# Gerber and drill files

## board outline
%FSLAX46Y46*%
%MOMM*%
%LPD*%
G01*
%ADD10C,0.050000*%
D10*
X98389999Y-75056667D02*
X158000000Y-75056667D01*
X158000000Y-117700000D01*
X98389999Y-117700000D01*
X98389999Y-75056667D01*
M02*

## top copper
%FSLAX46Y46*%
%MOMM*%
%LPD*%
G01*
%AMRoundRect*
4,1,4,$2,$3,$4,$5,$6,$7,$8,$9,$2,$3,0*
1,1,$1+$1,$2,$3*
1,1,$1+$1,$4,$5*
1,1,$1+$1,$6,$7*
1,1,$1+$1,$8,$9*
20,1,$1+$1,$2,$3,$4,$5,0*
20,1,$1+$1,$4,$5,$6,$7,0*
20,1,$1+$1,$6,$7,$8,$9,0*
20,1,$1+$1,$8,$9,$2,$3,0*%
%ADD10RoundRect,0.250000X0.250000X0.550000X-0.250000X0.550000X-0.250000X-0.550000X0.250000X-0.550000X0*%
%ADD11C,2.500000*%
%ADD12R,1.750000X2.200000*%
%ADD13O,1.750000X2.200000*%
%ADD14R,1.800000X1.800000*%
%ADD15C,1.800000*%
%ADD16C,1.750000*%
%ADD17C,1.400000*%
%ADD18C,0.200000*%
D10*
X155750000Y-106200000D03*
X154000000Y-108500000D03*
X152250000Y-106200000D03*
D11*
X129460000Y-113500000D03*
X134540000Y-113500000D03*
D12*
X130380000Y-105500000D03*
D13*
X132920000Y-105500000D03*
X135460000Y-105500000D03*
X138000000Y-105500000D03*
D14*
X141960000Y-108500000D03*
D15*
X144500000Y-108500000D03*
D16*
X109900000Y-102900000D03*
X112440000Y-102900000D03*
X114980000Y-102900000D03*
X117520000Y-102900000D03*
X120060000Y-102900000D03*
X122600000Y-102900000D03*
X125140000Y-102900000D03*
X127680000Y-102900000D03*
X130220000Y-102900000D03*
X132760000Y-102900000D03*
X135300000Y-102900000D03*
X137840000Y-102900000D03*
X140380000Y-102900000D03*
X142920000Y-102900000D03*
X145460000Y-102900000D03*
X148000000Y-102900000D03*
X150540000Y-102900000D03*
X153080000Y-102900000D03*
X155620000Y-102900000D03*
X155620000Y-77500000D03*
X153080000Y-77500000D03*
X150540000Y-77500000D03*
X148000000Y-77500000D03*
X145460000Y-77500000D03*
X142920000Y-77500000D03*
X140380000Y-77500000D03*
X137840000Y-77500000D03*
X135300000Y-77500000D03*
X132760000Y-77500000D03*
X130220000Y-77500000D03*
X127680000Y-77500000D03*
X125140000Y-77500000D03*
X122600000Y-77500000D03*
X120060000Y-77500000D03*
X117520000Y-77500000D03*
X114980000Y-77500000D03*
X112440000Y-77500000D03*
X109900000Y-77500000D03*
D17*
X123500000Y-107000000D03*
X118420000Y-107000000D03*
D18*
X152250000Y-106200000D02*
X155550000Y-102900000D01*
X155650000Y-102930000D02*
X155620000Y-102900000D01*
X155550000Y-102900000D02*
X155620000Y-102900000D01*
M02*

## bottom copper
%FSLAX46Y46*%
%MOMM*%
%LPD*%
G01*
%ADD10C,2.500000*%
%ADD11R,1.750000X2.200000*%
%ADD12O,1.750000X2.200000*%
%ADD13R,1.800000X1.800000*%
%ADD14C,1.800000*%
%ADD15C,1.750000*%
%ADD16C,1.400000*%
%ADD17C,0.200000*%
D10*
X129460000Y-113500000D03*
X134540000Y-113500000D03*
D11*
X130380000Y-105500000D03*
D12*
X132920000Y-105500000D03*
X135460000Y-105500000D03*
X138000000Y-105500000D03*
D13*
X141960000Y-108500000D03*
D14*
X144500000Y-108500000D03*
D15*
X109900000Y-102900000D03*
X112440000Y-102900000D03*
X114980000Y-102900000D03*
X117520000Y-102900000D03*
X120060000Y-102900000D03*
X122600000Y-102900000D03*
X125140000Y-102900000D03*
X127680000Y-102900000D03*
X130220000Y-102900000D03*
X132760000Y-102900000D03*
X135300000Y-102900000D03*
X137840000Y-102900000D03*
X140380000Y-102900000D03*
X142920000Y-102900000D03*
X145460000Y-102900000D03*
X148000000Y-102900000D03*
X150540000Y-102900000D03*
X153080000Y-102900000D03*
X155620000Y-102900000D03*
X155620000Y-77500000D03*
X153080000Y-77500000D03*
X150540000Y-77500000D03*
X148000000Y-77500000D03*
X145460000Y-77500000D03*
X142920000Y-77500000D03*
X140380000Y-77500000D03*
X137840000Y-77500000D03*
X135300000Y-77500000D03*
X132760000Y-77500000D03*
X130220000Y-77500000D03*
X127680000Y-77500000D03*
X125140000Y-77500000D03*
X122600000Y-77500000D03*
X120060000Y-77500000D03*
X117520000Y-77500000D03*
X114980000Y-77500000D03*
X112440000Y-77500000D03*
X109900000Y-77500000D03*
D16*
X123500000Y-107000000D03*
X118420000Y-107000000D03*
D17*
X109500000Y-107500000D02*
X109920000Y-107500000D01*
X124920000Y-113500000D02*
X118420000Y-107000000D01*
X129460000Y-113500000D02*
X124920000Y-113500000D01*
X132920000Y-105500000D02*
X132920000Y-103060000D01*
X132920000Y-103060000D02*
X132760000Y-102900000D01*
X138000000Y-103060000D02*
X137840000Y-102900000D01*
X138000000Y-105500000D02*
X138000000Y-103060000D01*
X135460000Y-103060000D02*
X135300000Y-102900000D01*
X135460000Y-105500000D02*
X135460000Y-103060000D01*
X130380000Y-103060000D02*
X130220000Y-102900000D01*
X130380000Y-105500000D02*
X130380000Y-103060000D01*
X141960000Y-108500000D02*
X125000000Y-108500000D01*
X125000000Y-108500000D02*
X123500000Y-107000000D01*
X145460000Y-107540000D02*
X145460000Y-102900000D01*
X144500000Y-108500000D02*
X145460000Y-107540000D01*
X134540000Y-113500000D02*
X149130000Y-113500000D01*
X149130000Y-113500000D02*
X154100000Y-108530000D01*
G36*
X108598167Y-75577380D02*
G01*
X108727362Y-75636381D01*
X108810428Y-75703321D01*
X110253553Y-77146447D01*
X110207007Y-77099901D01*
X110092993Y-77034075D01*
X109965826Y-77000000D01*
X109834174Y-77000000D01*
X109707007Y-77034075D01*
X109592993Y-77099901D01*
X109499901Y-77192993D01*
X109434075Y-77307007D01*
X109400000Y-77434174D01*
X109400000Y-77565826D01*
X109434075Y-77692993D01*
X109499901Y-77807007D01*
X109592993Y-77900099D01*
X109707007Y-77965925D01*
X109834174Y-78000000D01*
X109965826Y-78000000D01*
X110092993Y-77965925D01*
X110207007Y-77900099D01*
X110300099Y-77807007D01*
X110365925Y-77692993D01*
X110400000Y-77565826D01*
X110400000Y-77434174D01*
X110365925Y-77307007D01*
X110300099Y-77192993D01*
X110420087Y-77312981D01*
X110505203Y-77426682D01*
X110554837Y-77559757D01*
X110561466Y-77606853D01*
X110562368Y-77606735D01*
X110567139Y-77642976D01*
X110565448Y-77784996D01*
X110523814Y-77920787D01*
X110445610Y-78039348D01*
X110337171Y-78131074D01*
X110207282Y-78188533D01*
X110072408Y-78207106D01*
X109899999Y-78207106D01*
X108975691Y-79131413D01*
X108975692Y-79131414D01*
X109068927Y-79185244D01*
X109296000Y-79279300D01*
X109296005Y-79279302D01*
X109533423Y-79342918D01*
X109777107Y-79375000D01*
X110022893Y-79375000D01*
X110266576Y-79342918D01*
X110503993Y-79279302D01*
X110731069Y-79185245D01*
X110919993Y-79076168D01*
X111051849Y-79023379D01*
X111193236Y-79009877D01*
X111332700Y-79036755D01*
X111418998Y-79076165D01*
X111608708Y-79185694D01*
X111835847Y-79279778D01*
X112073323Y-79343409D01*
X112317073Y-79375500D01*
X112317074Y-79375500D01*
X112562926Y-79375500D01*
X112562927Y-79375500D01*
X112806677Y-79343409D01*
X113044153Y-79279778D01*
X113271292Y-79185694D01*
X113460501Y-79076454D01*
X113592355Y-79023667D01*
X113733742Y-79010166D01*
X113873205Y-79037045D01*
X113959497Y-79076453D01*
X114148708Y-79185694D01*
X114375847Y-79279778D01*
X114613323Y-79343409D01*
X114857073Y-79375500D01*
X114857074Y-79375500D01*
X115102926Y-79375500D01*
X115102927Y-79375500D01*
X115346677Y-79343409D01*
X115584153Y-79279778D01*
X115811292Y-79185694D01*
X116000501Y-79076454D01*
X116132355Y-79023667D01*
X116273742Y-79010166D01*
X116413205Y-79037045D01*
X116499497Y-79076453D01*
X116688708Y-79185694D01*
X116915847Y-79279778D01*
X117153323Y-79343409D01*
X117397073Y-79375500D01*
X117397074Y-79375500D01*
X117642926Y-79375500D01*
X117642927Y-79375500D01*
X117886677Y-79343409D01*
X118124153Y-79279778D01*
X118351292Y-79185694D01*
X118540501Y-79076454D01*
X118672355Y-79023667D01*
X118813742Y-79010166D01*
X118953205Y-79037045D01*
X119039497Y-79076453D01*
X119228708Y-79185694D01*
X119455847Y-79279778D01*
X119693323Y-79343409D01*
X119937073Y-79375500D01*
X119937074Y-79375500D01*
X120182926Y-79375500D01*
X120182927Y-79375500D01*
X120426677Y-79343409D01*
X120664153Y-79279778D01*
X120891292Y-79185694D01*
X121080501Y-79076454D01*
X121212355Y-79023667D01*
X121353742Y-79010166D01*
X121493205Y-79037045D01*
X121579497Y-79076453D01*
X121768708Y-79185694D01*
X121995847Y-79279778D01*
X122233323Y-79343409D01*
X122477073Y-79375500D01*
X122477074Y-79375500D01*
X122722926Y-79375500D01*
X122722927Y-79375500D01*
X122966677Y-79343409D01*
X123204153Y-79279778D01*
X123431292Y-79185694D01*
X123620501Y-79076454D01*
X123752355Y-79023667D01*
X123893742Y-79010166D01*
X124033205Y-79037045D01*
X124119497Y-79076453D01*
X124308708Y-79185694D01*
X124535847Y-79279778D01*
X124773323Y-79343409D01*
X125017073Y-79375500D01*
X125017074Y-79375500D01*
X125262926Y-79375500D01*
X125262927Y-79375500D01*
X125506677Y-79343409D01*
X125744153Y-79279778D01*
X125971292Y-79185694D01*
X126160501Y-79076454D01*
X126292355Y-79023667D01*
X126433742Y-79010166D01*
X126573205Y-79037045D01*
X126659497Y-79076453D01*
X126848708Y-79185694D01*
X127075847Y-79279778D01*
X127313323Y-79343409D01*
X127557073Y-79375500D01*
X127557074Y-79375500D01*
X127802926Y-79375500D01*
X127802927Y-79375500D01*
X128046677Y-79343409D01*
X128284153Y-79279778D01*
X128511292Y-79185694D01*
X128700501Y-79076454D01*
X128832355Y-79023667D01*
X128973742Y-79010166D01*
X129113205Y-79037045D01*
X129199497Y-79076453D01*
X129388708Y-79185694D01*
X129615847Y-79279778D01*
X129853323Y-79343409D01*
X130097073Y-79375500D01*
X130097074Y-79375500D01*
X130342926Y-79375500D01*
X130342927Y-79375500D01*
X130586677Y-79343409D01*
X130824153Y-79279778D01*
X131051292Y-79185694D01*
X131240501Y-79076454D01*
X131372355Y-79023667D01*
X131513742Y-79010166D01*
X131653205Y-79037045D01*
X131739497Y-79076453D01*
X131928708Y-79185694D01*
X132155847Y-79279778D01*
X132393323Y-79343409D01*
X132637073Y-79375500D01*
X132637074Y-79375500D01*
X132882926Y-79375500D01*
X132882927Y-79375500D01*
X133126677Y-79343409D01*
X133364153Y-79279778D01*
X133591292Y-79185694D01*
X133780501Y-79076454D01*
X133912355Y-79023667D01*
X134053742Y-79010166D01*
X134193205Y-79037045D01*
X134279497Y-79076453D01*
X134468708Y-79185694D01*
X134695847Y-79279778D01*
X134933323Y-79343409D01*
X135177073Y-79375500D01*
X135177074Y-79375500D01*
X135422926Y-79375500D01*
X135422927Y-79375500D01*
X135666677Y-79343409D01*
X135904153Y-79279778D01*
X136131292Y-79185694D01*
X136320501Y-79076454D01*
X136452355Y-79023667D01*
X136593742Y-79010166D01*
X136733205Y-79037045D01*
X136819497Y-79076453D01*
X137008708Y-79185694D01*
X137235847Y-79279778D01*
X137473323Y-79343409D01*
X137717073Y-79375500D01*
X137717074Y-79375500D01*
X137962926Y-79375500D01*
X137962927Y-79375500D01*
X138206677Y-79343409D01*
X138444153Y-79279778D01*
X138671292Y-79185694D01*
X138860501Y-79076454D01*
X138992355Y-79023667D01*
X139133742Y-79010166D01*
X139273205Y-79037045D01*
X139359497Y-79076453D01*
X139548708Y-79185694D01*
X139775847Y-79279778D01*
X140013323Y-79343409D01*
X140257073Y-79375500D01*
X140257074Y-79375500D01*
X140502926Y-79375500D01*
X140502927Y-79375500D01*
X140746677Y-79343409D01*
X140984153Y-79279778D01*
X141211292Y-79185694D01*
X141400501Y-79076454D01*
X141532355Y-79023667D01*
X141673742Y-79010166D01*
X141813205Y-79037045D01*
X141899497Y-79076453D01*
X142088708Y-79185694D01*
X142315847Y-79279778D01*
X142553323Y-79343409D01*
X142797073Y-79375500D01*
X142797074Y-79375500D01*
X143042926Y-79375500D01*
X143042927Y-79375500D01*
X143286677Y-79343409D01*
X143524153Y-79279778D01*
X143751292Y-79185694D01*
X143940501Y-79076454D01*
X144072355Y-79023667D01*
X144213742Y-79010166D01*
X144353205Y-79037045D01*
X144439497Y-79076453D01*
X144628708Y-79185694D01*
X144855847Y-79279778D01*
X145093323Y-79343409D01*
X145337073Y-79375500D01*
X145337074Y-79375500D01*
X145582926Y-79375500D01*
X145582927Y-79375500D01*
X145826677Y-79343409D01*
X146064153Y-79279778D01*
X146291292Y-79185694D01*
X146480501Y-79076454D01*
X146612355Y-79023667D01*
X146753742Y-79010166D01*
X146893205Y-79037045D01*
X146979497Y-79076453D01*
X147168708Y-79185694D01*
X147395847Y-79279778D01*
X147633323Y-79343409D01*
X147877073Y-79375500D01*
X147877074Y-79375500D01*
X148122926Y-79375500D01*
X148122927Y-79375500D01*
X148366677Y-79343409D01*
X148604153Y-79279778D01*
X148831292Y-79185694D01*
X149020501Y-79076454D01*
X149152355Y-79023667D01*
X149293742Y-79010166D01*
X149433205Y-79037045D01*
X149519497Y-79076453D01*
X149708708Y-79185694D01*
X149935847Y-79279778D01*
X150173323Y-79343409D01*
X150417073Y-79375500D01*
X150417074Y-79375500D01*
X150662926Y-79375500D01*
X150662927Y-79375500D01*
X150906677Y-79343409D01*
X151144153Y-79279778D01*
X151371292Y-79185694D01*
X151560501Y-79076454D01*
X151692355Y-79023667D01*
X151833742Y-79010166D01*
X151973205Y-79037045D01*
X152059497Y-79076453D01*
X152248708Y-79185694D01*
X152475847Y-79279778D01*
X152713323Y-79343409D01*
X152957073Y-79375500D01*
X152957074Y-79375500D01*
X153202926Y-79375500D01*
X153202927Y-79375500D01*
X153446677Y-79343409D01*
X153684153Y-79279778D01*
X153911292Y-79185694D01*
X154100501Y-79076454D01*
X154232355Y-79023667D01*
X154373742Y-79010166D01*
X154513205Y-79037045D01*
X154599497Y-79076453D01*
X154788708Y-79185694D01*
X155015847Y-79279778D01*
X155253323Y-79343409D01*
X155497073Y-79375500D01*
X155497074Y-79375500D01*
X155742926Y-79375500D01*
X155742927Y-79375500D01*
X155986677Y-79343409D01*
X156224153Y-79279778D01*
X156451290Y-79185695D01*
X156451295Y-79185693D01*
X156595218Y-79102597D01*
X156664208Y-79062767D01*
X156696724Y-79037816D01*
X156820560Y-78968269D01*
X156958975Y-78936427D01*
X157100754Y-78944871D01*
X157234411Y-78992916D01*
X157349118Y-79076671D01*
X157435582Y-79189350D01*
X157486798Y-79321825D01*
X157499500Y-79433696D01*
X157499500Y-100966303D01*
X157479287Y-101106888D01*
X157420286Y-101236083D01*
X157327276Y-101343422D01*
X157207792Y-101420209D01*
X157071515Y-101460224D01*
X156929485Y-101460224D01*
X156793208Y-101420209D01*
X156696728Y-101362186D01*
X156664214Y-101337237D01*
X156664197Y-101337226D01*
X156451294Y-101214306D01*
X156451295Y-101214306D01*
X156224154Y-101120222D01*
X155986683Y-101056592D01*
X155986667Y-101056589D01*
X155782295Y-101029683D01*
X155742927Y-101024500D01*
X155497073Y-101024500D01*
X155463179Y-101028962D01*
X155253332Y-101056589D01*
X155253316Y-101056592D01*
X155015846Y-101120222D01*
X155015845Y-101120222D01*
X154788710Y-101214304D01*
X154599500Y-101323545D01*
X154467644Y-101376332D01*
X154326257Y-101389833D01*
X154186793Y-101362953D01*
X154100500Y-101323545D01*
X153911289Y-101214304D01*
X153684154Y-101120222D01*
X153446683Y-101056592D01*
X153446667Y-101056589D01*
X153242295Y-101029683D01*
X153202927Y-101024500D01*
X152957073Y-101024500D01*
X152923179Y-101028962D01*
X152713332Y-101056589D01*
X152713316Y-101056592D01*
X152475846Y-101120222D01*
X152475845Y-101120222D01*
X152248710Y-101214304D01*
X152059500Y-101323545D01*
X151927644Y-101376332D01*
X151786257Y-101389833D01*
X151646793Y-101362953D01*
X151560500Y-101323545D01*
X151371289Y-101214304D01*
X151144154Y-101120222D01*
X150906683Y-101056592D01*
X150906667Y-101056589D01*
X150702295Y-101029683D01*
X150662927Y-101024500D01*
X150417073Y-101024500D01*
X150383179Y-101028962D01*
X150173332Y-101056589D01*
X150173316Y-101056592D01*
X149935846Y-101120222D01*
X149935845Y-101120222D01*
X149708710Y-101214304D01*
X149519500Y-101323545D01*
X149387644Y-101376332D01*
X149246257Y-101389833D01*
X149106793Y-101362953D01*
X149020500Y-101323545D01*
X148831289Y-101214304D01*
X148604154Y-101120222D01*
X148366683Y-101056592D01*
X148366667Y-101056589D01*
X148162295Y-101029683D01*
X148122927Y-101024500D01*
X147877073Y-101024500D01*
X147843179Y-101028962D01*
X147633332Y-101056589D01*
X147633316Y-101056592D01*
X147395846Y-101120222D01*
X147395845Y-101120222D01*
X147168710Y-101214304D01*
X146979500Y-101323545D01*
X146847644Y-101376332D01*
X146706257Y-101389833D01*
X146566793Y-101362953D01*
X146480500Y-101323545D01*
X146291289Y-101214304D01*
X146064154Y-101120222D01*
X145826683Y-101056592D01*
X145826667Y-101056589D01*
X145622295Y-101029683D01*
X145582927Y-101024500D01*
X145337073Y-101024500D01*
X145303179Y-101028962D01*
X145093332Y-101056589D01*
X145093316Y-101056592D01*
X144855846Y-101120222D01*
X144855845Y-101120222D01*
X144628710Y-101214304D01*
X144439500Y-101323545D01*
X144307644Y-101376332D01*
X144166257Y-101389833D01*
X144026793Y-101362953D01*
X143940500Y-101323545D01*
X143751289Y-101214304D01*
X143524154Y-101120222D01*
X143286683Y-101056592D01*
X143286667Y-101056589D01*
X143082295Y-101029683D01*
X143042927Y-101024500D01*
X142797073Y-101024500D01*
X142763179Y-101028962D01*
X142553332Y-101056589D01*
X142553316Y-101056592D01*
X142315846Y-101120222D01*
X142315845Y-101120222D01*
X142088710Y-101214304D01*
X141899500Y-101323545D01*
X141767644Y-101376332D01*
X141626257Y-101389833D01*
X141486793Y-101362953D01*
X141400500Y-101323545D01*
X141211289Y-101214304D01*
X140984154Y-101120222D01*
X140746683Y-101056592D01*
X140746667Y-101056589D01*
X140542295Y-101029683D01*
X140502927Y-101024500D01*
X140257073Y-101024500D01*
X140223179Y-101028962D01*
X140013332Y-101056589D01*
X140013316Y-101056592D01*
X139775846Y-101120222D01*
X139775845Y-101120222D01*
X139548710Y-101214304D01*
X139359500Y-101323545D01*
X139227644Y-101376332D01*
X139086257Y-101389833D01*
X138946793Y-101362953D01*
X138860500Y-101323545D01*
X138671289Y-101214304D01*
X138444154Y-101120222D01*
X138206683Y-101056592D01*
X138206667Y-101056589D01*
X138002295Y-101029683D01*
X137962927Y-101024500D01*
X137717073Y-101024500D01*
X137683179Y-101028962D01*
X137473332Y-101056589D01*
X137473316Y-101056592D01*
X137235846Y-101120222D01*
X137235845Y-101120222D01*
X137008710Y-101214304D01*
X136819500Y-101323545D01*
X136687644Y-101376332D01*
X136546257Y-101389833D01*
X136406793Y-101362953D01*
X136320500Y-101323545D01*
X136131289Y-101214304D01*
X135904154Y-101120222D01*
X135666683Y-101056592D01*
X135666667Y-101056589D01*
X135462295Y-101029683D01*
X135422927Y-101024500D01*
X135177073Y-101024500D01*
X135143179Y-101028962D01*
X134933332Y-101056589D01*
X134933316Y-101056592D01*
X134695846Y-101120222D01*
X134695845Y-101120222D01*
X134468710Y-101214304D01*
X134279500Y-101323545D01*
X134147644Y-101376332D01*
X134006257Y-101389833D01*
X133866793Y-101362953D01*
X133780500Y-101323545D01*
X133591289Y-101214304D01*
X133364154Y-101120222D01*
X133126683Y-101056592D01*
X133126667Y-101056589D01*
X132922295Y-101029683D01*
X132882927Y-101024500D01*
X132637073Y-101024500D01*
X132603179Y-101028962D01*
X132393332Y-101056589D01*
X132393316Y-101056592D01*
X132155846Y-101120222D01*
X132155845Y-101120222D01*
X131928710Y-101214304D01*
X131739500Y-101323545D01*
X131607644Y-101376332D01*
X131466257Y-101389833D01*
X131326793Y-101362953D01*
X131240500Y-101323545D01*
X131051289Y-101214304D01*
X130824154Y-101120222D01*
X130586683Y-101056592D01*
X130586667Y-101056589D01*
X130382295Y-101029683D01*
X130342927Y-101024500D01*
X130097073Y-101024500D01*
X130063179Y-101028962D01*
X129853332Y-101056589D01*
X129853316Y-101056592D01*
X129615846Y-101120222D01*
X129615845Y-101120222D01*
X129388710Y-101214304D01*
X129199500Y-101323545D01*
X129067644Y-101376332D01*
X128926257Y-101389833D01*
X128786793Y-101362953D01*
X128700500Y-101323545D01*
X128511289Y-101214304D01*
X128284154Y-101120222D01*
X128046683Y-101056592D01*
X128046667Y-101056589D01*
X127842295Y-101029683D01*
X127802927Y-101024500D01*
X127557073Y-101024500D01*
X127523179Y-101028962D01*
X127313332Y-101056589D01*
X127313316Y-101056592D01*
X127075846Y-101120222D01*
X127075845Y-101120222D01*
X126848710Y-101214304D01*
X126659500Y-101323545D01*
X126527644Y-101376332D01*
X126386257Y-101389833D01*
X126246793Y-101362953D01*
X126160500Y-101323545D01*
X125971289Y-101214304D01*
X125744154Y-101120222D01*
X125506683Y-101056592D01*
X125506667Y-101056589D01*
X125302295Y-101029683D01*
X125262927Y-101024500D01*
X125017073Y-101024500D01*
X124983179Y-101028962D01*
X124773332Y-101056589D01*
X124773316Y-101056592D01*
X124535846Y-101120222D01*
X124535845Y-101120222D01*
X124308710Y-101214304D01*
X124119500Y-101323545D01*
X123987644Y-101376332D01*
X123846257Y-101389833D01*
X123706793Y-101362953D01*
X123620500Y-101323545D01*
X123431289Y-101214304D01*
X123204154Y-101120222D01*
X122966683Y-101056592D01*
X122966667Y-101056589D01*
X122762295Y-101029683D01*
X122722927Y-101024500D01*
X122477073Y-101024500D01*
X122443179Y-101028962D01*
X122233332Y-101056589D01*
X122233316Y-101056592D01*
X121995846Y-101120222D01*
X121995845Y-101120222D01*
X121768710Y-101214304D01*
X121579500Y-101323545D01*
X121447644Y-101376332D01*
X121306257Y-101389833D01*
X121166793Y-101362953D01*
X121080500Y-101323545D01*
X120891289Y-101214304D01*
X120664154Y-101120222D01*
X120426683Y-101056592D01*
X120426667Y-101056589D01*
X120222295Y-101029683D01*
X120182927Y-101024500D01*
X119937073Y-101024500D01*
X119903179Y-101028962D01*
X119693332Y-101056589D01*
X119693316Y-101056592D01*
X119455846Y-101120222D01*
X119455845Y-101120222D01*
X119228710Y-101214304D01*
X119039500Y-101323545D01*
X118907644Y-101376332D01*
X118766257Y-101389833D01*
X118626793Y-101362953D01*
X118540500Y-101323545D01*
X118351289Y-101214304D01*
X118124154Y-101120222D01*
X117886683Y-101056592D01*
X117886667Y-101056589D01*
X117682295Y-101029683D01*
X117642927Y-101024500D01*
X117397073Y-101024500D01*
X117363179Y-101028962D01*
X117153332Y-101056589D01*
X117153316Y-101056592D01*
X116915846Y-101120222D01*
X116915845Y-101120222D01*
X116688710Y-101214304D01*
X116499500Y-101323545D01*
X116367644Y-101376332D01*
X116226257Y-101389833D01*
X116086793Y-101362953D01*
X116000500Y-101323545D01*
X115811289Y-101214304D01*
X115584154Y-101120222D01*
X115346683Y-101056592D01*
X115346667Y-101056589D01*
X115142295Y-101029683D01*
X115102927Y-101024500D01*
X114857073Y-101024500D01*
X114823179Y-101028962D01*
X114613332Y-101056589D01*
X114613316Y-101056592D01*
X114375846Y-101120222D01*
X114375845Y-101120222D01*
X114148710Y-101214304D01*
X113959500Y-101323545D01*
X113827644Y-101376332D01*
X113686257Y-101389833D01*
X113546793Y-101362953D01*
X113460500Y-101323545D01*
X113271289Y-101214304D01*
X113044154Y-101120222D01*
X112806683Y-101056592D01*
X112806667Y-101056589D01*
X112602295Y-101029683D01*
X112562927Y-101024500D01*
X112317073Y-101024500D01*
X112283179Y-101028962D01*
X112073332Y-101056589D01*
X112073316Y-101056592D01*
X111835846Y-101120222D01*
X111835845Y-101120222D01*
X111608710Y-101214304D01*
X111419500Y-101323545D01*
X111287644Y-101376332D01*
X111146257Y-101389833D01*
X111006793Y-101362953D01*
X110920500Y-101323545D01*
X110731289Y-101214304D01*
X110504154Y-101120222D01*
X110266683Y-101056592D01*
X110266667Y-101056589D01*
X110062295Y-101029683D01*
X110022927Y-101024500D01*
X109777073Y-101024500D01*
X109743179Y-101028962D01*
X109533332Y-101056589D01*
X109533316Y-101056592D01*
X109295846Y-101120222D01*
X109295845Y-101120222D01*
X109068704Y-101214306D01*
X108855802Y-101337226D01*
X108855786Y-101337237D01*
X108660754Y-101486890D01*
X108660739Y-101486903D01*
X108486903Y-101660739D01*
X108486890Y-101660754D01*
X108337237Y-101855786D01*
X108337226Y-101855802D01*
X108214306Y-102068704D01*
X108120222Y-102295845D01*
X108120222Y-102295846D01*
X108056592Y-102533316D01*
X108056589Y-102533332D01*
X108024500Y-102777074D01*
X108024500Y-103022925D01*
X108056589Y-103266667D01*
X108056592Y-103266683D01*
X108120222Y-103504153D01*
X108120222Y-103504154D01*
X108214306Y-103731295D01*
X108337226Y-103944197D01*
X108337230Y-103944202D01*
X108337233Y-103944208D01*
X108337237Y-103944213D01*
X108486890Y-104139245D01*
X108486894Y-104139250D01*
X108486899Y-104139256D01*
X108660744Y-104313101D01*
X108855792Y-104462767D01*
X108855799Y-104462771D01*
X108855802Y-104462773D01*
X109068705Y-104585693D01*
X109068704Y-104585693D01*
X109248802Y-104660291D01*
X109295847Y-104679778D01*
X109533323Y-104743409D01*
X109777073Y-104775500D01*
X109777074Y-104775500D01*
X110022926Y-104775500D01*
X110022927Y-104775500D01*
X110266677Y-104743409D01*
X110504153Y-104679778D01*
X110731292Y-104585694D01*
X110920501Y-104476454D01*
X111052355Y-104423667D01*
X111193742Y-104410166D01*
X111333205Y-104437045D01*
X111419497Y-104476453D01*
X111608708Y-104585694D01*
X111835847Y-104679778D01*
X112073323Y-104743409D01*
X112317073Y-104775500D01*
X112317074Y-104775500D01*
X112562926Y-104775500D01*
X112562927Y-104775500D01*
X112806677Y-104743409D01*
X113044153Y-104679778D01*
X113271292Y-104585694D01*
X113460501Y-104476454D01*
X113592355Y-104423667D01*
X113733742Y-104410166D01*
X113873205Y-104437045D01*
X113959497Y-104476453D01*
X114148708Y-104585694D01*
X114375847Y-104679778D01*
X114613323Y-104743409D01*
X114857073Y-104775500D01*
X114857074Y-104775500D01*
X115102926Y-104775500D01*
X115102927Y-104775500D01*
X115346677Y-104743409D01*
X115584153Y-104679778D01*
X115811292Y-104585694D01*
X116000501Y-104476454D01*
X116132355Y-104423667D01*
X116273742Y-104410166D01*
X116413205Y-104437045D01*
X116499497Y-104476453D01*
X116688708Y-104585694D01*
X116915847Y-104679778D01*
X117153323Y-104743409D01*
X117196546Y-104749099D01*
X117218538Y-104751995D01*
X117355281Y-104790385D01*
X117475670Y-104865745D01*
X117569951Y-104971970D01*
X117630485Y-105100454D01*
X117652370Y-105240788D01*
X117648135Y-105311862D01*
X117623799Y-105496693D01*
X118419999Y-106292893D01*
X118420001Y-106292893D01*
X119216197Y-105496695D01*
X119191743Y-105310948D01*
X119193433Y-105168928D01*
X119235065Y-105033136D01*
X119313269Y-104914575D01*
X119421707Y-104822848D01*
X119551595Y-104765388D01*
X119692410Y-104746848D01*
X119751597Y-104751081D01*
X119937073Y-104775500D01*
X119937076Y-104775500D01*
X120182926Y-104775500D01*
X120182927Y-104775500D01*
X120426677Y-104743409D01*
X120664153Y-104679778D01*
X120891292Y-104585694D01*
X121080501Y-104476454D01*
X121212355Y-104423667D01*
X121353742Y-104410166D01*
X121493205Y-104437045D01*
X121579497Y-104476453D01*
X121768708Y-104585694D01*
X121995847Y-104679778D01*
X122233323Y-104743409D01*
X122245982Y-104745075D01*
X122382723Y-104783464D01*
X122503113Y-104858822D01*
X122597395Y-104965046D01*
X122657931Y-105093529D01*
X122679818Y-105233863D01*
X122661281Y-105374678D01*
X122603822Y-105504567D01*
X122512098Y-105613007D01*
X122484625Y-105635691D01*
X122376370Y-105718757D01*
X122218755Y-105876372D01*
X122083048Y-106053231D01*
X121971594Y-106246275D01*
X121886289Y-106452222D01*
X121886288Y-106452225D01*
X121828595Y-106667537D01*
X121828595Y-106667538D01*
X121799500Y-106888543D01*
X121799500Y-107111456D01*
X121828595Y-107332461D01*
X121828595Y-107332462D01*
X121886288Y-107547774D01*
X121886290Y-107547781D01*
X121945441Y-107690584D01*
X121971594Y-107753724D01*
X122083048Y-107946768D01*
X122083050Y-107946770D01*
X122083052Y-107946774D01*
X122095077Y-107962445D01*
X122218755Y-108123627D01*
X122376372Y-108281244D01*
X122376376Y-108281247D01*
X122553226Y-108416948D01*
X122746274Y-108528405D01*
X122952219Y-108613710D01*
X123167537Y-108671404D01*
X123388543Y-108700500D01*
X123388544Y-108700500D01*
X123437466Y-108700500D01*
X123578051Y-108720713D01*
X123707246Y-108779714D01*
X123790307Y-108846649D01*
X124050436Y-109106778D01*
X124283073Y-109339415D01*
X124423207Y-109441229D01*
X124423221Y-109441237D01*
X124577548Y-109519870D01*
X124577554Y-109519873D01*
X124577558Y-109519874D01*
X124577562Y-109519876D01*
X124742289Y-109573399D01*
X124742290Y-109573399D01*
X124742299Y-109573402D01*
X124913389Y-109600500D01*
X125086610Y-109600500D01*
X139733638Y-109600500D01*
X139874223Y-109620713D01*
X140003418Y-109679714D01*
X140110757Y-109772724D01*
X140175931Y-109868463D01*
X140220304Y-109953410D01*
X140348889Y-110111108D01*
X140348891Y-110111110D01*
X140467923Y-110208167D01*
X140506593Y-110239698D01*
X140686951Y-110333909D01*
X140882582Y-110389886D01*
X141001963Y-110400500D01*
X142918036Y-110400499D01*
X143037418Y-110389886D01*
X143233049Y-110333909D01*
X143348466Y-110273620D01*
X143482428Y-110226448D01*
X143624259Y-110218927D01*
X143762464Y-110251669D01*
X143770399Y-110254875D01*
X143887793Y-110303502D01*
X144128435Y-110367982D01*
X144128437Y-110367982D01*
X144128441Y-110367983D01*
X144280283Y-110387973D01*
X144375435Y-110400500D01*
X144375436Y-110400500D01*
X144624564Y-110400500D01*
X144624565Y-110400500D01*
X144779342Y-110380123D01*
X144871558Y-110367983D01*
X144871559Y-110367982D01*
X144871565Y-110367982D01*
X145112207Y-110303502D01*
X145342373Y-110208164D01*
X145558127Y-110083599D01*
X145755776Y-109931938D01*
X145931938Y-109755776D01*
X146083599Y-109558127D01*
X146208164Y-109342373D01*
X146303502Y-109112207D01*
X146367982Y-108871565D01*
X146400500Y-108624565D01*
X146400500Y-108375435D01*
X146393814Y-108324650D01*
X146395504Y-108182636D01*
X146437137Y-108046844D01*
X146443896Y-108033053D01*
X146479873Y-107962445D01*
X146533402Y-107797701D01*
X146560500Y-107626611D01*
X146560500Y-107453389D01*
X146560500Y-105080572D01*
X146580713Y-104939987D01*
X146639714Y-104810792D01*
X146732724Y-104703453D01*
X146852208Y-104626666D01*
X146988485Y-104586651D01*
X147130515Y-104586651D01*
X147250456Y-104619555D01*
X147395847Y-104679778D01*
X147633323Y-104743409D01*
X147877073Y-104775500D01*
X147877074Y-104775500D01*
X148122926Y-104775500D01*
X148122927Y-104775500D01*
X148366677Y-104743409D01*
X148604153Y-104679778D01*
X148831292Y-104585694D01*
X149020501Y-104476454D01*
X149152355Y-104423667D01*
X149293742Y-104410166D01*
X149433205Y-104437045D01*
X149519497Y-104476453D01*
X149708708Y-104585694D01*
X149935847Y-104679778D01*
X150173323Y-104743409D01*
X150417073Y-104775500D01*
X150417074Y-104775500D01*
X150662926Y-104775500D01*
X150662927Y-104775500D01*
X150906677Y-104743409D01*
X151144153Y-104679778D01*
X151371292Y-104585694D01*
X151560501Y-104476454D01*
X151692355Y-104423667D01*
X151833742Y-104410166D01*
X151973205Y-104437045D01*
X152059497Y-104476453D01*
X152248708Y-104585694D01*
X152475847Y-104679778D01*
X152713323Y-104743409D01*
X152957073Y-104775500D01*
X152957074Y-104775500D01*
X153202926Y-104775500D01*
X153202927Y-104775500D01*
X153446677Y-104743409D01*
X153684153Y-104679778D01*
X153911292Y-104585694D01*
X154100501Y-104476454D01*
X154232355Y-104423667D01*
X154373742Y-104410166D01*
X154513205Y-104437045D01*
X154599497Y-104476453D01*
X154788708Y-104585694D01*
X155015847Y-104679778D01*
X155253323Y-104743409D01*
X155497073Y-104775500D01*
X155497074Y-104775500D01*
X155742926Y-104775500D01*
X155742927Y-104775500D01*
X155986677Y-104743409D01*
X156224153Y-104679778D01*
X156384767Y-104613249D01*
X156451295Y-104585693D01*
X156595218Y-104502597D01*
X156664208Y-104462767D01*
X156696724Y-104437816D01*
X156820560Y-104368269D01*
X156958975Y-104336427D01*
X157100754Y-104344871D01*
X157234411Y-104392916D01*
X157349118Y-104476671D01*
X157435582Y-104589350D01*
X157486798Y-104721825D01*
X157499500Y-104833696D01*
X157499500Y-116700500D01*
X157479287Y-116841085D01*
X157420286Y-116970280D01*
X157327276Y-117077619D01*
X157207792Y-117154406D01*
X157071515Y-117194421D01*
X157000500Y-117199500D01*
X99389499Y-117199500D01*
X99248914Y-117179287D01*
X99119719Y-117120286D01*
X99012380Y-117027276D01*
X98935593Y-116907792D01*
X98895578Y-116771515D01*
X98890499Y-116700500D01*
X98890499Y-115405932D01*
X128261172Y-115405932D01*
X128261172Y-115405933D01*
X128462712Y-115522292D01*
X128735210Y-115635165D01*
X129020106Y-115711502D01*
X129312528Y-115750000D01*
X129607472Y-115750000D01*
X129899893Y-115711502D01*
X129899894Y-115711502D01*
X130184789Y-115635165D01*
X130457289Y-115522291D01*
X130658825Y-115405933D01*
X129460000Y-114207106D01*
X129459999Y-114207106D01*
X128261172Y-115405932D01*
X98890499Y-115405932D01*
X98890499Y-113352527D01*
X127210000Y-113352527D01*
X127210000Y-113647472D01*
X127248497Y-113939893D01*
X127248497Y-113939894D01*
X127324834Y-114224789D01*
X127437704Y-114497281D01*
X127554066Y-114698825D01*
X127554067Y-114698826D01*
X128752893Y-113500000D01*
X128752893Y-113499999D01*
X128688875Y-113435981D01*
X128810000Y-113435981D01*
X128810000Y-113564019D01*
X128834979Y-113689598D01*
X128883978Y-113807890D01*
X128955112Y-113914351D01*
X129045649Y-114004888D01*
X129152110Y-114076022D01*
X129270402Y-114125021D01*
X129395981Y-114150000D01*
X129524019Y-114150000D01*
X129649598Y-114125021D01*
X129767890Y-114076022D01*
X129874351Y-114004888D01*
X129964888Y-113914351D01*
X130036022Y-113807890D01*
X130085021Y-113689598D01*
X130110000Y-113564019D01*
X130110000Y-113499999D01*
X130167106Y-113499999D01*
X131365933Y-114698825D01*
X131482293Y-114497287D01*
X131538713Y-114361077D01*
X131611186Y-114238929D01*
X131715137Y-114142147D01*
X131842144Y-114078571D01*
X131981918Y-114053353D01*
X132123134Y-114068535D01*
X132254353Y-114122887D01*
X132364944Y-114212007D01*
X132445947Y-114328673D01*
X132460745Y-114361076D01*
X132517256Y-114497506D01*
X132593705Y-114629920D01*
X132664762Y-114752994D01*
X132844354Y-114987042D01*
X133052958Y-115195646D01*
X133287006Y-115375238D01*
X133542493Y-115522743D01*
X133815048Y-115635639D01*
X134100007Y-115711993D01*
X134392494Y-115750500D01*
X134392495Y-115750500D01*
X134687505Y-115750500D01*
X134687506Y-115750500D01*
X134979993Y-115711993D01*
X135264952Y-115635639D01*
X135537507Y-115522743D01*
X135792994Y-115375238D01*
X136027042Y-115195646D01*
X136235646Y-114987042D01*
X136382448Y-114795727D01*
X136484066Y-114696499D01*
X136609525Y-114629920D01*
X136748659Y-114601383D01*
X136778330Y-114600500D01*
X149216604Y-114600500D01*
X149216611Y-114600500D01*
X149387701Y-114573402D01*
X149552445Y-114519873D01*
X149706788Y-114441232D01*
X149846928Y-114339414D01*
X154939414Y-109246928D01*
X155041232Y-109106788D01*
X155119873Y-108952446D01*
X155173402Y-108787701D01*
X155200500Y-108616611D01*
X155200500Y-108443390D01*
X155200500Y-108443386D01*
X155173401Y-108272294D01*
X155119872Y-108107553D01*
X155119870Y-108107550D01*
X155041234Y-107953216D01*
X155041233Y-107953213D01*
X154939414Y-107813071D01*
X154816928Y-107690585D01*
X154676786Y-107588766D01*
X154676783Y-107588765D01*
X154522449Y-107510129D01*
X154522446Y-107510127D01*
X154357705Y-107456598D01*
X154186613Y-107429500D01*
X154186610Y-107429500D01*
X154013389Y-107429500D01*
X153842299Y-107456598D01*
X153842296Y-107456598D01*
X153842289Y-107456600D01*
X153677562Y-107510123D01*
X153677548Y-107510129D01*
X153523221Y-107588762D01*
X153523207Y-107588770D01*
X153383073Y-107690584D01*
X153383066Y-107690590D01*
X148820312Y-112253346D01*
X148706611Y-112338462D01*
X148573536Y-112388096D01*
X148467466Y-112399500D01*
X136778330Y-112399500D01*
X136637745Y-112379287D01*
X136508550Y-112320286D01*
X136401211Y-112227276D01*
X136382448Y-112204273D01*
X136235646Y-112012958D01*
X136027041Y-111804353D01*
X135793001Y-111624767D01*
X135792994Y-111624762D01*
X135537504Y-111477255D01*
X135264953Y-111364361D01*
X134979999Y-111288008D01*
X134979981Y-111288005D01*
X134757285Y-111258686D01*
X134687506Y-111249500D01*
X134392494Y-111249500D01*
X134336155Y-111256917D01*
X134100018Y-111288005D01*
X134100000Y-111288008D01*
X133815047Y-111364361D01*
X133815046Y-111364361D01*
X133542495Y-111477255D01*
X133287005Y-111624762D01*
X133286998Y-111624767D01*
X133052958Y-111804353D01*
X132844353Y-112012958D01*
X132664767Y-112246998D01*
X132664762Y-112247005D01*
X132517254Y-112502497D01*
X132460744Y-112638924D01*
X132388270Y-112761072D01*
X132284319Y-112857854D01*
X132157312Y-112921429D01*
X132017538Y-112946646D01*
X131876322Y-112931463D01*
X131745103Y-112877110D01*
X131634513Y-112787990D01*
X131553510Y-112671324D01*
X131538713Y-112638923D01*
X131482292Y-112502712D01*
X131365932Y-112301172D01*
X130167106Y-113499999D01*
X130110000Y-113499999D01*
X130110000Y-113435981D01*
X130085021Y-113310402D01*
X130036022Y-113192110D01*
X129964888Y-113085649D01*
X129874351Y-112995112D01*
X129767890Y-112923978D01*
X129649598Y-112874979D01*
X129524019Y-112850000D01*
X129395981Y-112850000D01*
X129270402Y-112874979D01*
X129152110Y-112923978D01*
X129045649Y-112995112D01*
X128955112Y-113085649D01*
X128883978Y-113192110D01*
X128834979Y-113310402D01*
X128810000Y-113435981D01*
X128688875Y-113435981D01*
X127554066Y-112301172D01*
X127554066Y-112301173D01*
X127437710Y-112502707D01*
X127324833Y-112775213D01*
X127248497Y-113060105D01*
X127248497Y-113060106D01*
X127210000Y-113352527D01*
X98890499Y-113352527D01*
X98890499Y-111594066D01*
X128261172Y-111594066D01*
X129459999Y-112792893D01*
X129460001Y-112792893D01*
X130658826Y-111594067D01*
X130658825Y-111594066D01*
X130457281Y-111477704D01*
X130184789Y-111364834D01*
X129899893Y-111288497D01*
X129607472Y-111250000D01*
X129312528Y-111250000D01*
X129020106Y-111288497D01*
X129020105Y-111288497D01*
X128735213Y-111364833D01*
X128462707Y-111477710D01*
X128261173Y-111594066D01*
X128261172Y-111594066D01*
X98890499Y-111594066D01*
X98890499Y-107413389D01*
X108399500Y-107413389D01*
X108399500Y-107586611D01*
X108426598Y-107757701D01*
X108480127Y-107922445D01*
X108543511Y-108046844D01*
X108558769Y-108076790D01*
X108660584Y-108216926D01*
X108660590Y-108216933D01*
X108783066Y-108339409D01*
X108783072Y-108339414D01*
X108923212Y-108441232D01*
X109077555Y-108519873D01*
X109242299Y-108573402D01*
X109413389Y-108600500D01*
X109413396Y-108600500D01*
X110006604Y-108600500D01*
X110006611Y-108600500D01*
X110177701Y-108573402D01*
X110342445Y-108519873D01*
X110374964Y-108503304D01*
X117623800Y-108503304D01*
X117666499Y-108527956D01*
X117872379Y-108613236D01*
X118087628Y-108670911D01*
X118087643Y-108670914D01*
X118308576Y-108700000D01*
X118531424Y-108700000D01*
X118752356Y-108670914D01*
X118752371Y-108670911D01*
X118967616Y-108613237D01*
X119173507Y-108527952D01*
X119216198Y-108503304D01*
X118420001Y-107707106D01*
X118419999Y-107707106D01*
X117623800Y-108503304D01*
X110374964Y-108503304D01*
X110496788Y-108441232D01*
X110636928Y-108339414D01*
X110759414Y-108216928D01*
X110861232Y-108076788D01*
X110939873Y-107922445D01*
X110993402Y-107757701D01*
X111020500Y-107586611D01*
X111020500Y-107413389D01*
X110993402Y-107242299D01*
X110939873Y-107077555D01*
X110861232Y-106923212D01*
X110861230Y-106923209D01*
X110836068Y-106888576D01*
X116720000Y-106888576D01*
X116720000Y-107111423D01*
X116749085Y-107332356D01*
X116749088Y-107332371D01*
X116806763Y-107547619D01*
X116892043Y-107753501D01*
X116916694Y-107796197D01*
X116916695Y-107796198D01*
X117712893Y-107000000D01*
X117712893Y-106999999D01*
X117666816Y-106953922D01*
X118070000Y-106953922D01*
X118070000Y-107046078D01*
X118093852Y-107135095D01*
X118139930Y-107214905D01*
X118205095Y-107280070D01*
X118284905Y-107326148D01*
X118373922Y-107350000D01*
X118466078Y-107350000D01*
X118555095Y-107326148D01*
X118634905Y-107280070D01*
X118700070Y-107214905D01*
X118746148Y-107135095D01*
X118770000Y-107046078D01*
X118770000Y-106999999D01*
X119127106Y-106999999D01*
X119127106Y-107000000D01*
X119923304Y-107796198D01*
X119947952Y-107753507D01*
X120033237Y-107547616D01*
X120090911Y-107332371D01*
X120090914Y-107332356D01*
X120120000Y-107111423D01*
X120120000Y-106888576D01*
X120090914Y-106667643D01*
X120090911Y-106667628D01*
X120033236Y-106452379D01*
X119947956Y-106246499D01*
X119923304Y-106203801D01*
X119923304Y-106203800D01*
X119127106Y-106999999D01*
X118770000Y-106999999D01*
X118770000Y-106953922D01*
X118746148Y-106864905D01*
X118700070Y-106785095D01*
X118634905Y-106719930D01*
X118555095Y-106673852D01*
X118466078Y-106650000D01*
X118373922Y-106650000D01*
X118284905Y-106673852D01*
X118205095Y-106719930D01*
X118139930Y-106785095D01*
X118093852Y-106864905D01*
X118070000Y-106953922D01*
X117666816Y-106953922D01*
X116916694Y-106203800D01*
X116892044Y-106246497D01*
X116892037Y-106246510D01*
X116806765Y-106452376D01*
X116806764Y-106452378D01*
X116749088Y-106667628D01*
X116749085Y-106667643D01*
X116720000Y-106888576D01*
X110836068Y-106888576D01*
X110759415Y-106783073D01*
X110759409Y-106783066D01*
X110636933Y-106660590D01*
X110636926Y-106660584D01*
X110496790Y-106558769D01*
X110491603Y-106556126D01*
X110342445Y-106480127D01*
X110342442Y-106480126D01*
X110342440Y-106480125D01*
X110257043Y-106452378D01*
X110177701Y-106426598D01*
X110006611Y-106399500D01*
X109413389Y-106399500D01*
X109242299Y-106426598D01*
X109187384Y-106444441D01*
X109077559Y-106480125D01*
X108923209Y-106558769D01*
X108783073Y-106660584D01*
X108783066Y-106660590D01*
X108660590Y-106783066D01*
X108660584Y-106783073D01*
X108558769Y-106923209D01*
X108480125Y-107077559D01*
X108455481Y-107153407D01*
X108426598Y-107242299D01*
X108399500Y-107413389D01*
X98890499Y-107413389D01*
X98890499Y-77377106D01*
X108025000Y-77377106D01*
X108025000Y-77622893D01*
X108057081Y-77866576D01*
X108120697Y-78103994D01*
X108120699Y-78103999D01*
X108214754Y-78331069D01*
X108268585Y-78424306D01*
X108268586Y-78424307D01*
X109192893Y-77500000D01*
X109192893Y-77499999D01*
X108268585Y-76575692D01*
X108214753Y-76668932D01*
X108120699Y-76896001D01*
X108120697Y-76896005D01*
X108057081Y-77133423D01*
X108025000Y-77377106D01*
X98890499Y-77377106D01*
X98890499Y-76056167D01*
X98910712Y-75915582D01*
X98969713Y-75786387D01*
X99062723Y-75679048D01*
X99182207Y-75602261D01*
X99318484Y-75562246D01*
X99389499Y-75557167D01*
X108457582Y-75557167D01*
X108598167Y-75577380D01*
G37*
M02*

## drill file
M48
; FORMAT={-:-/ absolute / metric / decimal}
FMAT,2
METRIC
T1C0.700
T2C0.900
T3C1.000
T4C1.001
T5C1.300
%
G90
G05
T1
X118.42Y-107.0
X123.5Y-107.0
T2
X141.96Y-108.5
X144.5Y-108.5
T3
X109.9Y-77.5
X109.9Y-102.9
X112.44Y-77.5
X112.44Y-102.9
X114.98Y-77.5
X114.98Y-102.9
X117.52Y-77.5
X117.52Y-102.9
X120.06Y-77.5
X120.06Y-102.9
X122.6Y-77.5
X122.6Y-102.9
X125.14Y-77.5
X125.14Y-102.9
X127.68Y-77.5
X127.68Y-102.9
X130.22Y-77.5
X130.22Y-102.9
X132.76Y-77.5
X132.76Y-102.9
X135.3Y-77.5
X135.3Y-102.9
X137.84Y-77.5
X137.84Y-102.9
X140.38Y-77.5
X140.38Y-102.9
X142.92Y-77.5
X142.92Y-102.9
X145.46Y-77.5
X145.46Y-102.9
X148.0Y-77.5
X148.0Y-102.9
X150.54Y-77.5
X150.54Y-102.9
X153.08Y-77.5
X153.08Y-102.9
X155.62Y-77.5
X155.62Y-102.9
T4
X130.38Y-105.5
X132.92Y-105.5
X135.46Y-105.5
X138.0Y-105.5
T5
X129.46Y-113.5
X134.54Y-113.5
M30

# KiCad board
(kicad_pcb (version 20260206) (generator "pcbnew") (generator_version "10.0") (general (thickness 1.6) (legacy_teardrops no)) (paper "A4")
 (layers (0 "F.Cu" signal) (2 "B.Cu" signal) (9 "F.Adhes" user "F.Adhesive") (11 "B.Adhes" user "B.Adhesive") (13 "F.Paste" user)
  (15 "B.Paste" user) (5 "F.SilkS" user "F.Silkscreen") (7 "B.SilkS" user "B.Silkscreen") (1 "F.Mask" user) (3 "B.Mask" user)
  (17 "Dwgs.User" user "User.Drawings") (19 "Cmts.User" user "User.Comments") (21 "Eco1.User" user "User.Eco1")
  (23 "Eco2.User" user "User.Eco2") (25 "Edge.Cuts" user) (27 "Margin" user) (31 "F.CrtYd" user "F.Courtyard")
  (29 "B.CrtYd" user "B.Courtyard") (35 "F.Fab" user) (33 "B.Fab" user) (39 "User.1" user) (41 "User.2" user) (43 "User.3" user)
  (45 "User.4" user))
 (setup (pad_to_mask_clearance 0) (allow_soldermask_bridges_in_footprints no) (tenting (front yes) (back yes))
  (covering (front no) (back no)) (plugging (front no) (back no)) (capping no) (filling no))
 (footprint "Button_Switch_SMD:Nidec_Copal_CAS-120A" (layer "F.Cu") (at 154 107.35 -90)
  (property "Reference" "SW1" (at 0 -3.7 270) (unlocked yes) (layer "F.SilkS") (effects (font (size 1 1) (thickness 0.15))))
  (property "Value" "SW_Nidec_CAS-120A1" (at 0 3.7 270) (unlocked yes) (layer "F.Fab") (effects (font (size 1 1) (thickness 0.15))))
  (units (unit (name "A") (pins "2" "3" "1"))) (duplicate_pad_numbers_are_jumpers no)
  (pad "1" smd roundrect (at -1.15 -1.75 180) (size 1 1.6) (layers "F.Cu" "F.Mask" "F.Paste") (roundrect_rratio 0.25)
   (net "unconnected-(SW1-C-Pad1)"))
  (pad "2" smd roundrect (at 1.15 0 180) (size 1 1.6) (layers "F.Cu" "F.Mask" "F.Paste") (roundrect_rratio 0.25) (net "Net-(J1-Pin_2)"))
  (pad "3" smd roundrect (at -1.15 1.75 180) (size 1 1.6) (layers "F.Cu" "F.Mask" "F.Paste") (roundrect_rratio 0.25) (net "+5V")))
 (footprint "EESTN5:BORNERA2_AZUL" (layer "F.Cu") (at 132 113.5)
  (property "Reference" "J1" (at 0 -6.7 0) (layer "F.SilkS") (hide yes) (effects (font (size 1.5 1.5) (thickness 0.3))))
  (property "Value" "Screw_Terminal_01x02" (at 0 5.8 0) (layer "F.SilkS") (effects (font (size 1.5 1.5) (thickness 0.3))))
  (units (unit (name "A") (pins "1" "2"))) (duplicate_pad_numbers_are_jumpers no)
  (pad "1" thru_hole circle (at -2.54 0) (size 2.5 2.5) (drill 1.3) (layers "*.Cu" "*.Mask" "F.SilkS") (remove_unused_layers no) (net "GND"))
  (pad "2" thru_hole circle (at 2.54 0) (size 2.5 2.5) (drill 1.3) (layers "*.Cu" "*.Mask" "F.SilkS") (remove_unused_layers no)
   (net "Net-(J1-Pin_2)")))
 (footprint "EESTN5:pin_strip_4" (layer "F.Cu") (at 134.19 105.5)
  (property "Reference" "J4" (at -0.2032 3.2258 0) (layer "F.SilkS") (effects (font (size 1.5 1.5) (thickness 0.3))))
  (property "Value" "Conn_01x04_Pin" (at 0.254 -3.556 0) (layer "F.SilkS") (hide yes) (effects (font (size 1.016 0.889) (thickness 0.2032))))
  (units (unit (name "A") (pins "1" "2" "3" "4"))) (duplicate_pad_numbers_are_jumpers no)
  (pad "1" thru_hole rect (at -3.81 0) (size 1.75 2.2) (drill 1.00076) (layers "*.Cu" "*.Mask" "F.SilkS") (remove_unused_layers no)
   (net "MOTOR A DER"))
  (pad "2" thru_hole oval (at -1.27 0) (size 1.75 2.2) (drill 1.00076) (layers "*.Cu" "*.Mask" "F.SilkS") (remove_unused_layers no)
   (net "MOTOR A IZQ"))
  (pad "3" thru_hole oval (at 1.27 0) (size 1.75 2.2) (drill 1.00076) (layers "*.Cu" "*.Mask" "F.SilkS") (remove_unused_layers no)
   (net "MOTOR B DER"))
  (pad "4" thru_hole oval (at 3.81 0) (size 1.75 2.2) (drill 1.00076) (layers "*.Cu" "*.Mask" "F.SilkS") (remove_unused_layers no)
   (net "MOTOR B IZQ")))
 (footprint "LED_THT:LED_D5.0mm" (layer "F.Cu") (at 141.96 108.5)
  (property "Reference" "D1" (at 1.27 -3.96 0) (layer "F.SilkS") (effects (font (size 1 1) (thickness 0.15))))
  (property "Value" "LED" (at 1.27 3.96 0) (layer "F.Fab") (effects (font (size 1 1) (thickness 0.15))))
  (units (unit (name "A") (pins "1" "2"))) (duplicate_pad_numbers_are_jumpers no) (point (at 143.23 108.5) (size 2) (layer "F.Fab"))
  (pad "1" thru_hole rect (at 0 0) (size 1.8 1.8) (drill 0.9) (layers "*.Cu" "*.Mask") (remove_unused_layers no) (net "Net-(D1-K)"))
  (pad "2" thru_hole circle (at 2.54 0) (size 1.8 1.8) (drill 0.9) (layers "*.Cu" "*.Mask") (remove_unused_layers no) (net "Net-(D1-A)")))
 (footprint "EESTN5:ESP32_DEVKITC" (layer "F.Cu") (at 132.76 90.2)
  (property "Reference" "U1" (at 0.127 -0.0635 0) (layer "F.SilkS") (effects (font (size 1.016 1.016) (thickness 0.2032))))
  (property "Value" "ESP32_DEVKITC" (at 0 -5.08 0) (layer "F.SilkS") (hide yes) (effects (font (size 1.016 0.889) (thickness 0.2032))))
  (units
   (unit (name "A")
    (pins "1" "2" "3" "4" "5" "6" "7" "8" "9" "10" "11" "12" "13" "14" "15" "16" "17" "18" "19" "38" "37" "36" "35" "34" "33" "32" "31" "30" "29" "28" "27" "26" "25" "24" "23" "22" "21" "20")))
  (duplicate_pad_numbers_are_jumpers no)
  (pad "1" thru_hole circle (at -22.86 12.7) (size 1.75 1.75) (drill 1) (layers "*.Cu" "*.Mask" "F.SilkS") (remove_unused_layers no)
   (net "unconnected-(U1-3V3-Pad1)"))
  (pad "2" thru_hole circle (at -20.32 12.7) (size 1.75 1.75) (drill 1) (layers "*.Cu" "*.Mask" "F.SilkS") (remove_unused_layers no)
   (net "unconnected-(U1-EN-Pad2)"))
  (pad "3" thru_hole circle (at -17.78 12.7) (size 1.75 1.75) (drill 1) (layers "*.Cu" "*.Mask" "F.SilkS") (remove_unused_layers no)
   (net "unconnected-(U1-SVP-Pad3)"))
  (pad "4" thru_hole circle (at -15.24 12.7) (size 1.75 1.75) (drill 1) (layers "*.Cu" "*.Mask" "F.SilkS") (remove_unused_layers no)
   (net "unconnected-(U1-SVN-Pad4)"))
  (pad "5" thru_hole circle (at -12.7 12.7) (size 1.75 1.75) (drill 1) (layers "*.Cu" "*.Mask" "F.SilkS") (remove_unused_layers no)
   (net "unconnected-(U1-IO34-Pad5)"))
  (pad "6" thru_hole circle (at -10.16 12.7) (size 1.75 1.75) (drill 1) (layers "*.Cu" "*.Mask" "F.SilkS") (remove_unused_layers no)
   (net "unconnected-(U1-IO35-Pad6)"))
  (pad "7" thru_hole circle (at -7.62 12.7) (size 1.75 1.75) (drill 1) (layers "*.Cu" "*.Mask" "F.SilkS") (remove_unused_layers no)
   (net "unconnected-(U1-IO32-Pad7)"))
  (pad "8" thru_hole circle (at -5.08 12.7) (size 1.75 1.75) (drill 1) (layers "*.Cu" "*.Mask" "F.SilkS") (remove_unused_layers no)
   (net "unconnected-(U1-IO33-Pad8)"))
  (pad "9" thru_hole circle (at -2.54 12.7) (size 1.75 1.75) (drill 1) (layers "*.Cu" "*.Mask" "F.SilkS") (remove_unused_layers no)
   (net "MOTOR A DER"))
  (pad "10" thru_hole circle (at 0 12.7) (size 1.75 1.75) (drill 1) (layers "*.Cu" "*.Mask" "F.SilkS") (remove_unused_layers no)
   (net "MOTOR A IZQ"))
  (pad "11" thru_hole circle (at 2.54 12.7) (size 1.75 1.75) (drill 1) (layers "*.Cu" "*.Mask" "F.SilkS") (remove_unused_layers no)
   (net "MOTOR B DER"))
  (pad "12" thru_hole circle (at 5.08 12.7) (size 1.75 1.75) (drill 1) (layers "*.Cu" "*.Mask" "F.SilkS") (remove_unused_layers no)
   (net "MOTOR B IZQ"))
  (pad "13" thru_hole circle (at 7.62 12.7) (size 1.75 1.75) (drill 1) (layers "*.Cu" "*.Mask" "F.SilkS") (remove_unused_layers no)
   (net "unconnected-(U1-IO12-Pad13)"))
  (pad "14" thru_hole circle (at 10.16 12.7) (size 1.75 1.75) (drill 1) (layers "*.Cu" "*.Mask" "F.SilkS") (remove_unused_layers no)
   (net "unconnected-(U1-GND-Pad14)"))
  (pad "15" thru_hole circle (at 12.7 12.7) (size 1.75 1.75) (drill 1) (layers "*.Cu" "*.Mask" "F.SilkS") (remove_unused_layers no)
   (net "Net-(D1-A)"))
  (pad "16" thru_hole circle (at 15.24 12.7) (size 1.75 1.75) (drill 1) (layers "*.Cu" "*.Mask" "F.SilkS") (remove_unused_layers no)
   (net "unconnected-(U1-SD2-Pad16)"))
  (pad "17" thru_hole circle (at 17.78 12.7) (size 1.75 1.75) (drill 1) (layers "*.Cu" "*.Mask" "F.SilkS") (remove_unused_layers no)
   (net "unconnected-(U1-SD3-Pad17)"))
  (pad "18" thru_hole circle (at 20.32 12.7) (size 1.75 1.75) (drill 1) (layers "*.Cu" "*.Mask" "F.SilkS") (remove_unused_layers no)
   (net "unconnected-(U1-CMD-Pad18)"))
  (pad "19" thru_hole circle (at 22.86 12.7) (size 1.75 1.75) (drill 1) (layers "*.Cu" "*.Mask" "F.SilkS") (remove_unused_layers no)
   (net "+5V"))
  (pad "20" thru_hole circle (at 22.86 -12.7 180) (size 1.75 1.75) (drill 1) (layers "*.Cu" "*.Mask" "F.SilkS") (remove_unused_layers no)
   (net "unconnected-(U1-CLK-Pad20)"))
  (pad "21" thru_hole circle (at 20.32 -12.7 180) (size 1.75 1.75) (drill 1) (layers "*.Cu" "*.Mask" "F.SilkS") (remove_unused_layers no)
   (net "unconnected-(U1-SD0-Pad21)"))
  (pad "22" thru_hole circle (at 17.78 -12.7 180) (size 1.75 1.75) (drill 1) (layers "*.Cu" "*.Mask" "F.SilkS") (remove_unused_layers no)
   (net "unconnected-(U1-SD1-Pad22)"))
  (pad "23" thru_hole circle (at 15.24 -12.7 180) (size 1.75 1.75) (drill 1) (layers "*.Cu" "*.Mask" "F.SilkS") (remove_unused_layers no)
   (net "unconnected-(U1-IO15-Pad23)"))
  (pad "24" thru_hole circle (at 12.7 -12.7 180) (size 1.75 1.75) (drill 1) (layers "*.Cu" "*.Mask" "F.SilkS") (remove_unused_layers no)
   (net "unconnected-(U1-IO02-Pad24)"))
  (pad "25" thru_hole circle (at 10.16 -12.7 180) (size 1.75 1.75) (drill 1) (layers "*.Cu" "*.Mask" "F.SilkS") (remove_unused_layers no)
   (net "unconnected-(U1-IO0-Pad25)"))
  (pad "26" thru_hole circle (at 7.62 -12.7 180) (size 1.75 1.75) (drill 1) (layers "*.Cu" "*.Mask" "F.SilkS") (remove_unused_layers no)
   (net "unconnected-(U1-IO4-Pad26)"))
  (pad "27" thru_hole circle (at 5.08 -12.7 180) (size 1.75 1.75) (drill 1) (layers "*.Cu" "*.Mask" "F.SilkS") (remove_unused_layers no)
   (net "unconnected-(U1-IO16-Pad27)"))
  (pad "28" thru_hole circle (at 2.54 -12.7 180) (size 1.75 1.75) (drill 1) (layers "*.Cu" "*.Mask" "F.SilkS") (remove_unused_layers no)
   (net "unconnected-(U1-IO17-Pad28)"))
  (pad "29" thru_hole circle (at 0 -12.7 180) (size 1.75 1.75) (drill 1) (layers "*.Cu" "*.Mask" "F.SilkS") (remove_unused_layers no)
   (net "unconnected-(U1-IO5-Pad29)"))
  (pad "30" thru_hole circle (at -2.54 -12.7 180) (size 1.75 1.75) (drill 1) (layers "*.Cu" "*.Mask" "F.SilkS") (remove_unused_layers no)
   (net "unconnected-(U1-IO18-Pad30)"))
  (pad "31" thru_hole circle (at -5.08 -12.7 180) (size 1.75 1.75) (drill 1) (layers "*.Cu" "*.Mask" "F.SilkS") (remove_unused_layers no)
   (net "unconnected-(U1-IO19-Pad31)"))
  (pad "32" thru_hole circle (at -7.62 -12.7 180) (size 1.75 1.75) (drill 1) (layers "*.Cu" "*.Mask" "F.SilkS") (remove_unused_layers no)
   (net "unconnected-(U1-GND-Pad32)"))
  (pad "33" thru_hole circle (at -10.16 -12.7 180) (size 1.75 1.75) (drill 1) (layers "*.Cu" "*.Mask" "F.SilkS") (remove_unused_layers no)
   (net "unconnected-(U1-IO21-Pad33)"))
  (pad "34" thru_hole circle (at -12.7 -12.7 180) (size 1.75 1.75) (drill 1) (layers "*.Cu" "*.Mask" "F.SilkS") (remove_unused_layers no)
   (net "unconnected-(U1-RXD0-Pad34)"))
  (pad "35" thru_hole circle (at -15.24 -12.7 180) (size 1.75 1.75) (drill 1) (layers "*.Cu" "*.Mask" "F.SilkS") (remove_unused_layers no)
   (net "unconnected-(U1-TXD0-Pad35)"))
  (pad "36" thru_hole circle (at -17.78 -12.7 180) (size 1.75 1.75) (drill 1) (layers "*.Cu" "*.Mask" "F.SilkS") (remove_unused_layers no)
   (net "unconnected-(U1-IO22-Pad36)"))
  (pad "37" thru_hole circle (at -20.32 -12.7 180) (size 1.75 1.75) (drill 1) (layers "*.Cu" "*.Mask" "F.SilkS") (remove_unused_layers no)
   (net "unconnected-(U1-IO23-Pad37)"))
  (pad "38" thru_hole circle (at -22.86 -12.7 180) (size 1.75 1.75) (drill 1) (layers "*.Cu" "*.Mask" "F.SilkS") (remove_unused_layers no)
   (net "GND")))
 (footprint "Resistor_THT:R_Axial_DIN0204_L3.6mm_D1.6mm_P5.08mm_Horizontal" (layer "F.Cu") (at 123.5 107 180)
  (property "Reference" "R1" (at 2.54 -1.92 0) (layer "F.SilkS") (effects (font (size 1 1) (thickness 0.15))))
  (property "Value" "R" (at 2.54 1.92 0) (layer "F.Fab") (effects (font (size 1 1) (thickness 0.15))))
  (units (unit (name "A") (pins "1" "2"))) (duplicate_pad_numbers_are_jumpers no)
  (pad "1" thru_hole circle (at 0 0 180) (size 1.4 1.4) (drill 0.7) (layers "*.Cu" "*.Mask") (remove_unused_layers no) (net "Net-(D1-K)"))
  (pad "2" thru_hole circle (at 5.08 0 180) (size 1.4 1.4) (drill 0.7) (layers "*.Cu" "*.Mask") (remove_unused_layers no) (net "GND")))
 (gr_rect (start 98.389999 75.056667) (end 158 117.7) (stroke (width 0.05) (type default)) (fill no) (layer "Edge.Cuts"))
 (segment (start 109.5 107.5) (end 109.92 107.5) (width 0.2) (layer "B.Cu") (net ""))
 (segment (start 152.25 106.2) (end 155.55 102.9) (width 0.2) (layer "F.Cu") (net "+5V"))
 (segment (start 155.65 102.93) (end 155.62 102.9) (width 0.2) (layer "F.Cu") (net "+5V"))
 (segment (start 155.55 102.9) (end 155.62 102.9) (width 0.2) (layer "F.Cu") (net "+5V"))
 (segment (start 124.92 113.5) (end 118.42 107) (width 0.2) (layer "B.Cu") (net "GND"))
 (segment (start 129.46 113.5) (end 124.92 113.5) (width 0.2) (layer "B.Cu") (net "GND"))
 (segment (start 132.92 105.5) (end 132.92 103.06) (width 0.2) (layer "B.Cu") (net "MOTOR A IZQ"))
 (segment (start 132.92 103.06) (end 132.76 102.9) (width 0.2) (layer "B.Cu") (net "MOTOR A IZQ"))
 (segment (start 138 103.06) (end 137.84 102.9) (width 0.2) (layer "B.Cu") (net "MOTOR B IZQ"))
 (segment (start 138 105.5) (end 138 103.06) (width 0.2) (layer "B.Cu") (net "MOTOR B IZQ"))
 (segment (start 135.46 103.06) (end 135.3 102.9) (width 0.2) (layer "B.Cu") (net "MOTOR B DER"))
 (segment (start 135.46 105.5) (end 135.46 103.06) (width 0.2) (layer "B.Cu") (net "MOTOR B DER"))
 (segment (start 130.38 103.06) (end 130.22 102.9) (width 0.2) (layer "B.Cu") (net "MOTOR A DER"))
 (segment (start 130.38 105.5) (end 130.38 103.06) (width 0.2) (layer "B.Cu") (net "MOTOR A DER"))
 (segment (start 141.96 108.5) (end 125 108.5) (width 0.2) (layer "B.Cu") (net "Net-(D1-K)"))
 (segment (start 125 108.5) (end 123.5 107) (width 0.2) (layer "B.Cu") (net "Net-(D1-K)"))
 (segment (start 145.46 107.54) (end 145.46 102.9) (width 0.2) (layer "B.Cu") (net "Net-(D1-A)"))
 (segment (start 144.5 108.5) (end 145.46 107.54) (width 0.2) (layer "B.Cu") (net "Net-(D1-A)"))
 (segment (start 134.54 113.5) (end 149.13 113.5) (width 0.2) (layer "B.Cu") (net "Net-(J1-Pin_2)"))
 (segment (start 149.13 113.5) (end 154.1 108.53) (width 0.2) (layer "B.Cu") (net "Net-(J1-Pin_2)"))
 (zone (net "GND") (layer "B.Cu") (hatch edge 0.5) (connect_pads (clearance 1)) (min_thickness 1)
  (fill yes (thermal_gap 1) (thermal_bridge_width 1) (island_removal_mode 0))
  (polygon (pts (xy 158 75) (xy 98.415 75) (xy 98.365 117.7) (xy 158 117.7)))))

